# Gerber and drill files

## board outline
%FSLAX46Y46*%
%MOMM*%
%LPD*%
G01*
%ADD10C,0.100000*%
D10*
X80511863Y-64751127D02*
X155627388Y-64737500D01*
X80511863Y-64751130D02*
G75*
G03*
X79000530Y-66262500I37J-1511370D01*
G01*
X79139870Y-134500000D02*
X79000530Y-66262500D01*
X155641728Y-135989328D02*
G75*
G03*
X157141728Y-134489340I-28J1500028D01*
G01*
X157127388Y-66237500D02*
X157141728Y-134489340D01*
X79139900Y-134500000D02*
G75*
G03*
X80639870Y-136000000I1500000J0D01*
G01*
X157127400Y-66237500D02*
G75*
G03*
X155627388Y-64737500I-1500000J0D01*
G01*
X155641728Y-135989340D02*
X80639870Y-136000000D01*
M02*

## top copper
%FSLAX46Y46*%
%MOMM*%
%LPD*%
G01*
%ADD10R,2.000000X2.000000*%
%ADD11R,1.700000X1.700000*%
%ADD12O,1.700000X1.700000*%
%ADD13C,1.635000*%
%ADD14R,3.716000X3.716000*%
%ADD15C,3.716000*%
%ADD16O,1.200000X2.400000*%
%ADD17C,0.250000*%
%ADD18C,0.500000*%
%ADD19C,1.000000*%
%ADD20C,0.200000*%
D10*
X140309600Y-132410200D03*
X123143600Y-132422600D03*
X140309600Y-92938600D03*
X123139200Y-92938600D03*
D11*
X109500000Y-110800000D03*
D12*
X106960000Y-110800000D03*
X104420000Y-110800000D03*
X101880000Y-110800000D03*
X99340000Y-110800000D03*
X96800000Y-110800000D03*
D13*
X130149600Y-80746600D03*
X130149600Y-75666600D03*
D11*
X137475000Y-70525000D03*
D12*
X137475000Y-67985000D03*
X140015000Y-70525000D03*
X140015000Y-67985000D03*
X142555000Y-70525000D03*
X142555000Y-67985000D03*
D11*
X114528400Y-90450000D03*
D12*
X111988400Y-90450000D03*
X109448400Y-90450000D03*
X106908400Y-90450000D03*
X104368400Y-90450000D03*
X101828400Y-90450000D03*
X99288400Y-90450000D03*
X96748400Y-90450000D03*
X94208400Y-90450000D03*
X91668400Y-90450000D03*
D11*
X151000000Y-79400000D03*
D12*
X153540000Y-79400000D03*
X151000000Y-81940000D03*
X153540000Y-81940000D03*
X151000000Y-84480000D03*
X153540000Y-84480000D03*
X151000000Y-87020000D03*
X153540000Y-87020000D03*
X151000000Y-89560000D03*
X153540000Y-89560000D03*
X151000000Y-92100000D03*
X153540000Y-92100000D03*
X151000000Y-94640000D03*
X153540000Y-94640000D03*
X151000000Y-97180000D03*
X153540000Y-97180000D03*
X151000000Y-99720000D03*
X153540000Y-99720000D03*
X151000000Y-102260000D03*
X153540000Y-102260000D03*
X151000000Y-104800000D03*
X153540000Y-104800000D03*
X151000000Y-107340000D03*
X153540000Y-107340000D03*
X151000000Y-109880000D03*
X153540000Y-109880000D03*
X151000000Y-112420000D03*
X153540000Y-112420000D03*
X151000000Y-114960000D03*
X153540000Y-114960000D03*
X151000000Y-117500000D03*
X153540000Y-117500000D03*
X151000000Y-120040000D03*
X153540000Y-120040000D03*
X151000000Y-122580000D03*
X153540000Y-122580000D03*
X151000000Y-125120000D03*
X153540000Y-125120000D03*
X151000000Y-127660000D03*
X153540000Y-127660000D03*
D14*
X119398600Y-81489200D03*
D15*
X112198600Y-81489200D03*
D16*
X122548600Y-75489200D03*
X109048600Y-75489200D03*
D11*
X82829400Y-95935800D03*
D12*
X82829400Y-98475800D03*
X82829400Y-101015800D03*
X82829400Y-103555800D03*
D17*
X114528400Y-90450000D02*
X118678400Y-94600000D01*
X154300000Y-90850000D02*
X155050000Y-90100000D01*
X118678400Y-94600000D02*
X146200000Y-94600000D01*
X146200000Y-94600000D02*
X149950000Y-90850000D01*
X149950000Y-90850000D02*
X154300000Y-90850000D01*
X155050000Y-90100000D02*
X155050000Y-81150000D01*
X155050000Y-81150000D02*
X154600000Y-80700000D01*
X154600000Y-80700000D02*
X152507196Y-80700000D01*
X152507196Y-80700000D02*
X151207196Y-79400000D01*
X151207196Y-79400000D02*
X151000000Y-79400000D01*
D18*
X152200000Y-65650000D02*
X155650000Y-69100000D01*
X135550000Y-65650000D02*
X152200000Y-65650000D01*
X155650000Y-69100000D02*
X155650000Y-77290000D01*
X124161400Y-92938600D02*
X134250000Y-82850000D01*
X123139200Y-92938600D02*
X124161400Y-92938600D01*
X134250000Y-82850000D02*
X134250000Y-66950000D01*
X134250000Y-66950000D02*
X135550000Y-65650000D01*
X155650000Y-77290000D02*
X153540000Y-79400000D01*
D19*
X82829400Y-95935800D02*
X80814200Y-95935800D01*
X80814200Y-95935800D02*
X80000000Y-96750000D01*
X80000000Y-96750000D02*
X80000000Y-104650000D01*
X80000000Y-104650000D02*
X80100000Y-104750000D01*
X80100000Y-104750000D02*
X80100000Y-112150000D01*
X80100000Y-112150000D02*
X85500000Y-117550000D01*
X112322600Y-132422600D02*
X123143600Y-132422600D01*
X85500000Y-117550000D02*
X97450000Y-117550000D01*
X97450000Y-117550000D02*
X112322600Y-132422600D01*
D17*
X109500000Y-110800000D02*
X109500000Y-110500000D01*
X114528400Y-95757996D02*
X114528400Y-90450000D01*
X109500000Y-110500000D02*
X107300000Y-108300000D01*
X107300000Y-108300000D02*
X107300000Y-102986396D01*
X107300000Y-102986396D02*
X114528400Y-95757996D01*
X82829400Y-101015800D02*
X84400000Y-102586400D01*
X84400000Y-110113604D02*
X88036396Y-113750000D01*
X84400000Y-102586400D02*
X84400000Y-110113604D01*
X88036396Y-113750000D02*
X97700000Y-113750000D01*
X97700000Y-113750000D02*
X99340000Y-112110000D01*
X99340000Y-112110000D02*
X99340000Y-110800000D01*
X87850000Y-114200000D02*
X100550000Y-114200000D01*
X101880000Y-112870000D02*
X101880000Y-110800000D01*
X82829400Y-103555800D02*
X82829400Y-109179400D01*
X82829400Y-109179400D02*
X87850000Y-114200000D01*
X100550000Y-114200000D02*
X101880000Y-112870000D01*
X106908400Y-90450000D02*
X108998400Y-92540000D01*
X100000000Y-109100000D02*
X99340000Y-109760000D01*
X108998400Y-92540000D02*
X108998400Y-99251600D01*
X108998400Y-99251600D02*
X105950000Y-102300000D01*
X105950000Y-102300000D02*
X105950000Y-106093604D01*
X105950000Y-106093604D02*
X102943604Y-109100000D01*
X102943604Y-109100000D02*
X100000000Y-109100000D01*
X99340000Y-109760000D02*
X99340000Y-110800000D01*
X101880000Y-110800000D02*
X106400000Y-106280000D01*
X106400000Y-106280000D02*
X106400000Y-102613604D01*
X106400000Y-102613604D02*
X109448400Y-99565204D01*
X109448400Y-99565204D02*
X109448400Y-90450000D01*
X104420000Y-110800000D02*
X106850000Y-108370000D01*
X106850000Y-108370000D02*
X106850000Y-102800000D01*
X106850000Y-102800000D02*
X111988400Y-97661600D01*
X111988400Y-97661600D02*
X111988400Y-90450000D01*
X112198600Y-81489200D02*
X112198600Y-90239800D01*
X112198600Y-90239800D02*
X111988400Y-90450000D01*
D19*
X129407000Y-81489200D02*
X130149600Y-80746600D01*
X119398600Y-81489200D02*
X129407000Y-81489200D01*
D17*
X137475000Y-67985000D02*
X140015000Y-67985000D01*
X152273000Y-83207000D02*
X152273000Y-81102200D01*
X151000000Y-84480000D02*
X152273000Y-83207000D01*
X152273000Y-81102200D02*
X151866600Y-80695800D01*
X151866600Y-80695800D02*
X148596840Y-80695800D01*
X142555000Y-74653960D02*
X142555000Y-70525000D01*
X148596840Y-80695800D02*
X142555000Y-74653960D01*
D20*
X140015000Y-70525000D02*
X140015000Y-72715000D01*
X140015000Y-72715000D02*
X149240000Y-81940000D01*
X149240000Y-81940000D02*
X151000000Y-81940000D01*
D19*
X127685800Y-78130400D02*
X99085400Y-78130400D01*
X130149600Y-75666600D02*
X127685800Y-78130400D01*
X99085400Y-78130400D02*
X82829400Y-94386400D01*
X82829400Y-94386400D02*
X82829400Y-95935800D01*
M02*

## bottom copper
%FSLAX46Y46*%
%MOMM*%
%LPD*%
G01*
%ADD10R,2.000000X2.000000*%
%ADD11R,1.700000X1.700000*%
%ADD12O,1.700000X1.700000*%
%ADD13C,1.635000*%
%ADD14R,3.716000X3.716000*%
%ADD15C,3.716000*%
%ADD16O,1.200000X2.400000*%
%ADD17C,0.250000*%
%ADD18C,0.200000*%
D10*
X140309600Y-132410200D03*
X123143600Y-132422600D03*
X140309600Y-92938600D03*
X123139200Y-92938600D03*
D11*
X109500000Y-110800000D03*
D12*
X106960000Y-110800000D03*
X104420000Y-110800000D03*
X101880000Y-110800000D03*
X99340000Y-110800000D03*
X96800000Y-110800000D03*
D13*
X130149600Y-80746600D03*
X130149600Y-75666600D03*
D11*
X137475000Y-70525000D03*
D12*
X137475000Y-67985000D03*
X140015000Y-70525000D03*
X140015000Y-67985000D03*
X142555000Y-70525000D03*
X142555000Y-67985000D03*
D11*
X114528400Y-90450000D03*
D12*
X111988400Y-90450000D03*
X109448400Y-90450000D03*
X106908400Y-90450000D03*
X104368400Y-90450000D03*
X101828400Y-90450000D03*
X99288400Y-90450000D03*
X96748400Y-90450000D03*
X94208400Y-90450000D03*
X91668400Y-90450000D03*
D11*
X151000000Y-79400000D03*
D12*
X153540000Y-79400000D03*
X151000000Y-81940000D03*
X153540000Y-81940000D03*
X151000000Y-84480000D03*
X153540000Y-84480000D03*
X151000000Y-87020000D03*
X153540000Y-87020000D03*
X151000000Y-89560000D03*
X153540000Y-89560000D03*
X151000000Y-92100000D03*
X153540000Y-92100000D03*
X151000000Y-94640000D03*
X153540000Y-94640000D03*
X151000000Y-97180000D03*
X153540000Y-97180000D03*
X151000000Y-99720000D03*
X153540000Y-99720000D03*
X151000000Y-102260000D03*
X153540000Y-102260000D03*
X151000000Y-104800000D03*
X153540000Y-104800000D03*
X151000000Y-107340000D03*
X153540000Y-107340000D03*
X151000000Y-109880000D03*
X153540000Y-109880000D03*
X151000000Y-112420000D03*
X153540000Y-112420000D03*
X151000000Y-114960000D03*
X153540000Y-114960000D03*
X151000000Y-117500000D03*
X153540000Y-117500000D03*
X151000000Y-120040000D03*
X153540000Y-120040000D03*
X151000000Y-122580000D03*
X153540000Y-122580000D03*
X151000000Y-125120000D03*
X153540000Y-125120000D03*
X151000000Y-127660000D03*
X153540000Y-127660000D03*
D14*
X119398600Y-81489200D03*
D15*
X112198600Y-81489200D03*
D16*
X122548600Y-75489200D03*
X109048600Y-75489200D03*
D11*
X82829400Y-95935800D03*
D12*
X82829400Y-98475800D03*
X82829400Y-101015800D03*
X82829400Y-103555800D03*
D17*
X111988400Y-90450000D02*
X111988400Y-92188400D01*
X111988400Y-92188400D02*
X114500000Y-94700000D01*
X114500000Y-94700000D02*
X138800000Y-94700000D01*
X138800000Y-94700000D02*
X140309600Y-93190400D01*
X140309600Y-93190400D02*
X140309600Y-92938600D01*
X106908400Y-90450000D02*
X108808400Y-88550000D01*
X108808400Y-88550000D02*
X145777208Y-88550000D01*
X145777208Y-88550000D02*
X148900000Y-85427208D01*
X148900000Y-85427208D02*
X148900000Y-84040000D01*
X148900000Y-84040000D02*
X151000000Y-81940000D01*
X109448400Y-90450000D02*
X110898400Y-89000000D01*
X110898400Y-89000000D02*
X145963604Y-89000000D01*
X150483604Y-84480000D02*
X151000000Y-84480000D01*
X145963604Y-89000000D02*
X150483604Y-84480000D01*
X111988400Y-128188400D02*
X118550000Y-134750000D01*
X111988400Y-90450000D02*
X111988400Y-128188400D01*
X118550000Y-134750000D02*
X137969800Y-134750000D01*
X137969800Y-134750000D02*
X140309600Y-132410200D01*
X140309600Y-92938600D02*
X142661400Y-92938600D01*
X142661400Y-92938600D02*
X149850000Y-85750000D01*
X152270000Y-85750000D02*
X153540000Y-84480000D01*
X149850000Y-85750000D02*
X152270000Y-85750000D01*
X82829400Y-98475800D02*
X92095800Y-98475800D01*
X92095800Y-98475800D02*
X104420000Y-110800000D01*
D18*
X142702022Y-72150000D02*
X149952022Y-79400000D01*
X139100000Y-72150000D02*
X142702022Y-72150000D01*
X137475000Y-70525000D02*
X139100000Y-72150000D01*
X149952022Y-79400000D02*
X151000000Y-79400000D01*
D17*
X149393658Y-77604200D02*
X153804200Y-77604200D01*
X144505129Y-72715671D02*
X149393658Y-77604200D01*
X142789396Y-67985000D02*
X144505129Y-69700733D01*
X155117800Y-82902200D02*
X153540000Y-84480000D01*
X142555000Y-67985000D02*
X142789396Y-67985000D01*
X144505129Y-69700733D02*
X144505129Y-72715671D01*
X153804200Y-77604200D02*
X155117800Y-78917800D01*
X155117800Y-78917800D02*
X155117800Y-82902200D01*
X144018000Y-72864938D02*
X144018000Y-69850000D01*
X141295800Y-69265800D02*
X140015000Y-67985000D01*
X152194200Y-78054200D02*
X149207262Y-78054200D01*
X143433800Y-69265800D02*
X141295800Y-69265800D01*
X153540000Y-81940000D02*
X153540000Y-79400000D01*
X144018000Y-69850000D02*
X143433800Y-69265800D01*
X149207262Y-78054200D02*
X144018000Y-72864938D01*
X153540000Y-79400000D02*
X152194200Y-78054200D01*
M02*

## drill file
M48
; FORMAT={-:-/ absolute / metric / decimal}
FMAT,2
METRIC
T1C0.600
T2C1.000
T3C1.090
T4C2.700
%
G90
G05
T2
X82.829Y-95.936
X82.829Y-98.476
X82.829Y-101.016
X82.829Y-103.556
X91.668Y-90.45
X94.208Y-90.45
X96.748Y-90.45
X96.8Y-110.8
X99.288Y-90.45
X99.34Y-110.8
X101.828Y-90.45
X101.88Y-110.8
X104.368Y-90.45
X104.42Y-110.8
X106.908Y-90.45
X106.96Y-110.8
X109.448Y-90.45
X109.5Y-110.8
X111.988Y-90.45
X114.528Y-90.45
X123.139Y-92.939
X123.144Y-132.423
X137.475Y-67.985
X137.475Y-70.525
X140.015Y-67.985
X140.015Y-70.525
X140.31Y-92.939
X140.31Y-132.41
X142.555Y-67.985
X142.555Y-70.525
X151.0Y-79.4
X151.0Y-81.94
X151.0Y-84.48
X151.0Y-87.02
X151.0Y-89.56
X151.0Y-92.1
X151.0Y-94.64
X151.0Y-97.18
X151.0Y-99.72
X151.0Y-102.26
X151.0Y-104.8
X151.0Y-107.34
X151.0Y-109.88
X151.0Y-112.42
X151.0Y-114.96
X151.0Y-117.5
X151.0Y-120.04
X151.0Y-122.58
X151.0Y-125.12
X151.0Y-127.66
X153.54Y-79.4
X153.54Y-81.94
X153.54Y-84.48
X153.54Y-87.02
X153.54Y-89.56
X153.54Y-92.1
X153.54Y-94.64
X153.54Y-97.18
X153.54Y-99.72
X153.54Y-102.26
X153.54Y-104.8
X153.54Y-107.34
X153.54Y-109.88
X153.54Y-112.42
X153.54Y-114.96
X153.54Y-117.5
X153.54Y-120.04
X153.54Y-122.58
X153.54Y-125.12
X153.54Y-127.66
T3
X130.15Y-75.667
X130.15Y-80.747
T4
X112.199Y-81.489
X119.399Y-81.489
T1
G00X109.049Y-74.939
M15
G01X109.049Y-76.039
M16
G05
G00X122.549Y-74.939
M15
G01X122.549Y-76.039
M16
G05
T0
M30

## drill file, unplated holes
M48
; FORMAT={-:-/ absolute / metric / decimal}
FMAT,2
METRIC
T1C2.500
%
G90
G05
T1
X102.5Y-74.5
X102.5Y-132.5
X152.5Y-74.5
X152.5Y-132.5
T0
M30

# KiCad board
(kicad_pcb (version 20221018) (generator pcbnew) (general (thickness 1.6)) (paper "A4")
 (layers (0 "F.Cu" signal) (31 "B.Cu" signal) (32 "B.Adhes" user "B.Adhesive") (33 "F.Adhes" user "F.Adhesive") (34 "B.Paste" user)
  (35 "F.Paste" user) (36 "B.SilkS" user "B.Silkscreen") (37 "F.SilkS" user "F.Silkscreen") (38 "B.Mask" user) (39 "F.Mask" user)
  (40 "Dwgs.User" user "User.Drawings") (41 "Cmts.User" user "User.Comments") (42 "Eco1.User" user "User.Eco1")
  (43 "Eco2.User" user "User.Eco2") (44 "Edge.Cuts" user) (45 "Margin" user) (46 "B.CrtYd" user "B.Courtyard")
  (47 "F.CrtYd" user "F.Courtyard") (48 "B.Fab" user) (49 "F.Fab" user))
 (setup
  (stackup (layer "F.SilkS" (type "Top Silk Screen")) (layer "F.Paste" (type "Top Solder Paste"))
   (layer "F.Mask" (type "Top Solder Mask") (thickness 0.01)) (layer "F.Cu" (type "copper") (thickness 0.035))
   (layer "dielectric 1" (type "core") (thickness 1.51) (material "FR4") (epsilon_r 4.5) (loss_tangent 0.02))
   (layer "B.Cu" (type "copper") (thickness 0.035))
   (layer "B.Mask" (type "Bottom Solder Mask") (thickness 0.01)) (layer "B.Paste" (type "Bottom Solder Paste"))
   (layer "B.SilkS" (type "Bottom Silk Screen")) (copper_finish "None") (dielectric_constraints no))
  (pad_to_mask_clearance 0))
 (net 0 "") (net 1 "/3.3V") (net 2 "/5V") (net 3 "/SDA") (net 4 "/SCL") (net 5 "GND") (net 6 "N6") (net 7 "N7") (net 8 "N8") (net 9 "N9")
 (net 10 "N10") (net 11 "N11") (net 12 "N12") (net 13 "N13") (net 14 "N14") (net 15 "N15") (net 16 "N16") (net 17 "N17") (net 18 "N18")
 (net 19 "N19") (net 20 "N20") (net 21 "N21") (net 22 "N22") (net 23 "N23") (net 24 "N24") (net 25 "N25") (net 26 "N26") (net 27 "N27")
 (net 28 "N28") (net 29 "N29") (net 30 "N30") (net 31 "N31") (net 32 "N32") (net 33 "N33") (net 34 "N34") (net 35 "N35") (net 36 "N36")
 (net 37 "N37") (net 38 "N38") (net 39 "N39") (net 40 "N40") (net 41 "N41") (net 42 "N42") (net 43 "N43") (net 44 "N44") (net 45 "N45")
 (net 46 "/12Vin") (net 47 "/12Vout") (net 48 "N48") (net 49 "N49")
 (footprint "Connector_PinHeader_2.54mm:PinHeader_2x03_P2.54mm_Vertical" (layer "F.Cu") (at 137.475 70.525 90)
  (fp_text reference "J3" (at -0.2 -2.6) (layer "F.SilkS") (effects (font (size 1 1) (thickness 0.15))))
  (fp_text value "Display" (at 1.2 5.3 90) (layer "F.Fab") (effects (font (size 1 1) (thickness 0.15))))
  (pad "1" thru_hole rect (at 0 0 90) (size 1.7 1.7) (drill 1) (layers "*.Cu" "*.Mask") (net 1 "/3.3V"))
  (pad "2" thru_hole oval (at 2.54 0 90) (size 1.7 1.7) (drill 1) (layers "*.Cu" "*.Mask") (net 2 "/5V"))
  (pad "3" thru_hole oval (at 0 2.54 90) (size 1.7 1.7) (drill 1) (layers "*.Cu" "*.Mask") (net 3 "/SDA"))
  (pad "4" thru_hole oval (at 2.54 2.54 90) (size 1.7 1.7) (drill 1) (layers "*.Cu" "*.Mask") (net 2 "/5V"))
  (pad "5" thru_hole oval (at 0 5.08 90) (size 1.7 1.7) (drill 1) (layers "*.Cu" "*.Mask") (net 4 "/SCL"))
  (pad "6" thru_hole oval (at 2.54 5.08 90) (size 1.7 1.7) (drill 1) (layers "*.Cu" "*.Mask") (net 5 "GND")))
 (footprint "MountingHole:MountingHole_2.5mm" (layer "F.Cu") (at 152.5 74.5)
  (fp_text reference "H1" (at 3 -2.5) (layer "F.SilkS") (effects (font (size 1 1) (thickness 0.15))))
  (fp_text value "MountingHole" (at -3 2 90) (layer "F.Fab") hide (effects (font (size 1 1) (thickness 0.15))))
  (pad "" np_thru_hole circle (at 0 0) (size 2.5 2.5) (drill 2.5) (layers "*.Cu" "*.Mask")))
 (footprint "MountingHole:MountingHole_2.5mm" (layer "F.Cu") (at 102.5 74.5)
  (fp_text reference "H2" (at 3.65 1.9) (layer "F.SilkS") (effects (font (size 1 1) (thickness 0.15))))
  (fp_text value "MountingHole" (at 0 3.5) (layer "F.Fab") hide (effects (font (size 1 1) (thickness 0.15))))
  (pad "" np_thru_hole circle (at 0 0) (size 2.5 2.5) (drill 2.5) (layers "*.Cu" "*.Mask")))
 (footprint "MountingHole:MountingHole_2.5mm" (layer "F.Cu") (at 102.5 132.5)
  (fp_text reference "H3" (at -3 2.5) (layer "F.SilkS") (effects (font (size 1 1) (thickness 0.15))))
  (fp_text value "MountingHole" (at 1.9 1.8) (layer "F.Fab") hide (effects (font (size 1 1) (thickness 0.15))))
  (pad "" np_thru_hole circle (at 0 0) (size 2.5 2.5) (drill 2.5) (layers "*.Cu" "*.Mask")))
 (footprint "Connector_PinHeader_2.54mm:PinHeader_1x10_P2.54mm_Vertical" (layer "F.Cu") (at 114.5284 90.45 -90)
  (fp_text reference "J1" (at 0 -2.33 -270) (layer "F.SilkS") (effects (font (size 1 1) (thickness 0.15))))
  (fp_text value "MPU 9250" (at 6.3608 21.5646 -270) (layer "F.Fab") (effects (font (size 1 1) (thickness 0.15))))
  (pad "1" thru_hole rect (at 0 0 270) (size 1.7 1.7) (drill 1) (layers "*.Cu" "*.Mask") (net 1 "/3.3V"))
  (pad "2" thru_hole oval (at 0 2.54 270) (size 1.7 1.7) (drill 1) (layers "*.Cu" "*.Mask") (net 5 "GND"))
  (pad "3" thru_hole oval (at 0 5.08 270) (size 1.7 1.7) (drill 1) (layers "*.Cu" "*.Mask") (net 4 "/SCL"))
  (pad "4" thru_hole oval (at 0 7.62 270) (size 1.7 1.7) (drill 1) (layers "*.Cu" "*.Mask") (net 3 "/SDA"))
  (pad "5" thru_hole oval (at 0 10.16 270) (size 1.7 1.7) (drill 1) (layers "*.Cu" "*.Mask") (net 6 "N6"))
  (pad "6" thru_hole oval (at 0 12.7 270) (size 1.7 1.7) (drill 1) (layers "*.Cu" "*.Mask") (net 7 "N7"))
  (pad "7" thru_hole oval (at 0 15.24 270) (size 1.7 1.7) (drill 1) (layers "*.Cu" "*.Mask") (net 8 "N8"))
  (pad "8" thru_hole oval (at 0 17.78 270) (size 1.7 1.7) (drill 1) (layers "*.Cu" "*.Mask") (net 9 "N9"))
  (pad "9" thru_hole oval (at 0 20.32 270) (size 1.7 1.7) (drill 1) (layers "*.Cu" "*.Mask") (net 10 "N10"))
  (pad "10" thru_hole oval (at 0 22.86 270) (size 1.7 1.7) (drill 1) (layers "*.Cu" "*.Mask") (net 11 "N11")))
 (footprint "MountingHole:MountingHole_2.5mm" (layer "F.Cu") (at 152.5 132.5)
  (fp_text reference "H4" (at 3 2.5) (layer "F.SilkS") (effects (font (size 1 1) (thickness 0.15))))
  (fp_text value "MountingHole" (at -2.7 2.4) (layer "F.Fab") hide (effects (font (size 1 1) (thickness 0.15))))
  (pad "" np_thru_hole circle (at 0 0) (size 2.5 2.5) (drill 2.5) (layers "*.Cu" "*.Mask")))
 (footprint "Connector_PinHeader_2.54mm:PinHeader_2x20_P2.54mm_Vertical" (layer "F.Cu") (at 151 79.4)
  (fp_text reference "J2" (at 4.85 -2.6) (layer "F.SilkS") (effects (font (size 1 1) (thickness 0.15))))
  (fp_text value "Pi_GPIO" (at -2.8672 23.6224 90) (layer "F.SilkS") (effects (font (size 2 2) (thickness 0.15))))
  (pad "1" thru_hole rect (at 0 0) (size 1.7 1.7) (drill 1) (layers "*.Cu" "*.Mask") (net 1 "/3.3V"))
  (pad "2" thru_hole oval (at 2.54 0) (size 1.7 1.7) (drill 1) (layers "*.Cu" "*.Mask") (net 2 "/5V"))
  (pad "3" thru_hole oval (at 0 2.54) (size 1.7 1.7) (drill 1) (layers "*.Cu" "*.Mask") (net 3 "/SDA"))
  (pad "4" thru_hole oval (at 2.54 2.54) (size 1.7 1.7) (drill 1) (layers "*.Cu" "*.Mask") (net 2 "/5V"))
  (pad "5" thru_hole oval (at 0 5.08) (size 1.7 1.7) (drill 1) (layers "*.Cu" "*.Mask") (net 4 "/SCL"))
  (pad "6" thru_hole oval (at 2.54 5.08) (size 1.7 1.7) (drill 1) (layers "*.Cu" "*.Mask") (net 5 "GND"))
  (pad "7" thru_hole oval (at 0 7.62) (size 1.7 1.7) (drill 1) (layers "*.Cu" "*.Mask") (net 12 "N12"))
  (pad "8" thru_hole oval (at 2.54 7.62) (size 1.7 1.7) (drill 1) (layers "*.Cu" "*.Mask") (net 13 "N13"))
  (pad "9" thru_hole oval (at 0 10.16) (size 1.7 1.7) (drill 1) (layers "*.Cu" "*.Mask") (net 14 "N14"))
  (pad "10" thru_hole oval (at 2.54 10.16) (size 1.7 1.7) (drill 1) (layers "*.Cu" "*.Mask") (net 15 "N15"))
  (pad "11" thru_hole oval (at 0 12.7) (size 1.7 1.7) (drill 1) (layers "*.Cu" "*.Mask") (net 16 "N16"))
  (pad "12" thru_hole oval (at 2.54 12.7) (size 1.7 1.7) (drill 1) (layers "*.Cu" "*.Mask") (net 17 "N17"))
  (pad "13" thru_hole oval (at 0 15.24) (size 1.7 1.7) (drill 1) (layers "*.Cu" "*.Mask") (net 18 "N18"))
  (pad "14" thru_hole oval (at 2.54 15.24) (size 1.7 1.7) (drill 1) (layers "*.Cu" "*.Mask") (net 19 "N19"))
  (pad "15" thru_hole oval (at 0 17.78) (size 1.7 1.7) (drill 1) (layers "*.Cu" "*.Mask") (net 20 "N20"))
  (pad "16" thru_hole oval (at 2.54 17.78) (size 1.7 1.7) (drill 1) (layers "*.Cu" "*.Mask") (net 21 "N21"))
  (pad "17" thru_hole oval (at 0 20.32) (size 1.7 1.7) (drill 1) (layers "*.Cu" "*.Mask") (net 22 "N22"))
  (pad "18" thru_hole oval (at 2.54 20.32) (size 1.7 1.7) (drill 1) (layers "*.Cu" "*.Mask") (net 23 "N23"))
  (pad "19" thru_hole oval (at 0 22.86) (size 1.7 1.7) (drill 1) (layers "*.Cu" "*.Mask") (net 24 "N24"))
  (pad "20" thru_hole oval (at 2.54 22.86) (size 1.7 1.7) (drill 1) (layers "*.Cu" "*.Mask") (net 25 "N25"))
  (pad "21" thru_hole oval (at 0 25.4) (size 1.7 1.7) (drill 1) (layers "*.Cu" "*.Mask") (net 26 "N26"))
  (pad "22" thru_hole oval (at 2.54 25.4) (size 1.7 1.7) (drill 1) (layers "*.Cu" "*.Mask") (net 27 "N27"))
  (pad "23" thru_hole oval (at 0 27.94) (size 1.7 1.7) (drill 1) (layers "*.Cu" "*.Mask") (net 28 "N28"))
  (pad "24" thru_hole oval (at 2.54 27.94) (size 1.7 1.7) (drill 1) (layers "*.Cu" "*.Mask") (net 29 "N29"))
  (pad "25" thru_hole oval (at 0 30.48) (size 1.7 1.7) (drill 1) (layers "*.Cu" "*.Mask") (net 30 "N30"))
  (pad "26" thru_hole oval (at 2.54 30.48) (size 1.7 1.7) (drill 1) (layers "*.Cu" "*.Mask") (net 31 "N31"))
  (pad "27" thru_hole oval (at 0 33.02) (size 1.7 1.7) (drill 1) (layers "*.Cu" "*.Mask") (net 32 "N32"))
  (pad "28" thru_hole oval (at 2.54 33.02) (size 1.7 1.7) (drill 1) (layers "*.Cu" "*.Mask") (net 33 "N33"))
  (pad "29" thru_hole oval (at 0 35.56) (size 1.7 1.7) (drill 1) (layers "*.Cu" "*.Mask") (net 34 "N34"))
  (pad "30" thru_hole oval (at 2.54 35.56) (size 1.7 1.7) (drill 1) (layers "*.Cu" "*.Mask") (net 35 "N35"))
  (pad "31" thru_hole oval (at 0 38.1) (size 1.7 1.7) (drill 1) (layers "*.Cu" "*.Mask") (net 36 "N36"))
  (pad "32" thru_hole oval (at 2.54 38.1) (size 1.7 1.7) (drill 1) (layers "*.Cu" "*.Mask") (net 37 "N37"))
  (pad "33" thru_hole oval (at 0 40.64) (size 1.7 1.7) (drill 1) (layers "*.Cu" "*.Mask") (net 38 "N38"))
  (pad "34" thru_hole oval (at 2.54 40.64) (size 1.7 1.7) (drill 1) (layers "*.Cu" "*.Mask") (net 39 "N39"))
  (pad "35" thru_hole oval (at 0 43.18) (size 1.7 1.7) (drill 1) (layers "*.Cu" "*.Mask") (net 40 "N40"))
  (pad "36" thru_hole oval (at 2.54 43.18) (size 1.7 1.7) (drill 1) (layers "*.Cu" "*.Mask") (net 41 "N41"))
  (pad "37" thru_hole oval (at 0 45.72) (size 1.7 1.7) (drill 1) (layers "*.Cu" "*.Mask") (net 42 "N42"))
  (pad "38" thru_hole oval (at 2.54 45.72) (size 1.7 1.7) (drill 1) (layers "*.Cu" "*.Mask") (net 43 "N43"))
  (pad "39" thru_hole oval (at 0 48.26) (size 1.7 1.7) (drill 1) (layers "*.Cu" "*.Mask") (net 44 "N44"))
  (pad "40" thru_hole oval (at 2.54 48.26) (size 1.7 1.7) (drill 1) (layers "*.Cu" "*.Mask") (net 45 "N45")))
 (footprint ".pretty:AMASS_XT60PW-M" (layer "F.Cu") (at 115.7986 75.4892)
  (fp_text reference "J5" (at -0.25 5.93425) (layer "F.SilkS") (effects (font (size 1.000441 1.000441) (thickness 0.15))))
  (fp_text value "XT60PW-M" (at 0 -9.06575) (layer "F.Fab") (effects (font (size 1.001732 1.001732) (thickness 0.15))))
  (pad "1" thru_hole rect (at 3.6 6) (size 3.716 3.716) (drill 2.7) (layers "*.Cu" "*.Mask") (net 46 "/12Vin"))
  (pad "2" thru_hole circle (at -3.6 6) (size 3.716 3.716) (drill 2.7) (layers "*.Cu" "*.Mask") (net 5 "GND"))
  (pad "S1" thru_hole oval (at 6.75 0) (size 1.2 2.4) (drill oval 0.6 1.7) (layers "*.Cu" "*.Mask"))
  (pad "S2" thru_hole oval (at -6.75 0) (size 1.2 2.4) (drill oval 0.6 1.7) (layers "*.Cu" "*.Mask")))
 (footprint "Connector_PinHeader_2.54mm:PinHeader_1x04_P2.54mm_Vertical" (layer "F.Cu") (at 82.8294 95.9358)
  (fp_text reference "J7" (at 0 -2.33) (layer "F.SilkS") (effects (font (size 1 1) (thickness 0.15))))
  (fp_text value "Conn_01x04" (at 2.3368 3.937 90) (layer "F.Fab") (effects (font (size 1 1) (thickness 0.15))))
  (pad "1" thru_hole rect (at 0 0) (size 1.7 1.7) (drill 1) (layers "*.Cu" "*.Mask") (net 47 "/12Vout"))
  (pad "2" thru_hole oval (at 0 2.54) (size 1.7 1.7) (drill 1) (layers "*.Cu" "*.Mask") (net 5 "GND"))
  (pad "3" thru_hole oval (at 0 5.08) (size 1.7 1.7) (drill 1) (layers "*.Cu" "*.Mask") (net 3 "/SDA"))
  (pad "4" thru_hole oval (at 0 7.62) (size 1.7 1.7) (drill 1) (layers "*.Cu" "*.Mask") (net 4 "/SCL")))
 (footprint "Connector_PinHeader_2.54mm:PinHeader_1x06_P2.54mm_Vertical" (layer "F.Cu") (at 109.5 110.8 -90)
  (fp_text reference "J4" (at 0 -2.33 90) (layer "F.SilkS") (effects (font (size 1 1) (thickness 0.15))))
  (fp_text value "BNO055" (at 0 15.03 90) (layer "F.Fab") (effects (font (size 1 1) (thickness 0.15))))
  (pad "1" thru_hole rect (at 0 0 270) (size 1.7 1.7) (drill 1) (layers "*.Cu" "*.Mask") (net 1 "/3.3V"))
  (pad "2" thru_hole oval (at 0 2.54 270) (size 1.7 1.7) (drill 1) (layers "*.Cu" "*.Mask") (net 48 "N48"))
  (pad "3" thru_hole oval (at 0 5.08 270) (size 1.7 1.7) (drill 1) (layers "*.Cu" "*.Mask") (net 5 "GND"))
  (pad "4" thru_hole oval (at 0 7.62 270) (size 1.7 1.7) (drill 1) (layers "*.Cu" "*.Mask") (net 4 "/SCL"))
  (pad "5" thru_hole oval (at 0 10.16 270) (size 1.7 1.7) (drill 1) (layers "*.Cu" "*.Mask") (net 3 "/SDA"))
  (pad "6" thru_hole oval (at 0 12.7 270) (size 1.7 1.7) (drill 1) (layers "*.Cu" "*.Mask") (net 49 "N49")))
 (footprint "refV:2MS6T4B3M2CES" (layer "F.Cu") (at 130.1496 80.7466)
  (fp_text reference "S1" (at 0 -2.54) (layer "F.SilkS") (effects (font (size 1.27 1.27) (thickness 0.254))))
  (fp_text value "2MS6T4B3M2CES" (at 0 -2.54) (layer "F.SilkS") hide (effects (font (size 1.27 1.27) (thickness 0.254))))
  (pad "1" thru_hole circle (at 0 0) (size 1.635 1.635) (drill 1.09) (layers "*.Cu" "*.Mask") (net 46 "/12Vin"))
  (pad "3" thru_hole circle (at 0 -5.08) (size 1.635 1.635) (drill 1.09) (layers "*.Cu" "*.Mask") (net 47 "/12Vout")))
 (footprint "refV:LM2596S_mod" (layer "B.Cu") (at 145.6436 123.6726 90)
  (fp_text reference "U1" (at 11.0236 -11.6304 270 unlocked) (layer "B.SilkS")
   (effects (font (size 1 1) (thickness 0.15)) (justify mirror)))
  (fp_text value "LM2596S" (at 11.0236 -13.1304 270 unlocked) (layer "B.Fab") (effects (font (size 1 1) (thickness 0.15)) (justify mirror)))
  (pad "1" thru_hole rect (at -8.7376 -5.334 90) (size 2 2) (drill 1) (layers "*.Cu" "*.Mask") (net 5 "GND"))
  (pad "2" thru_hole rect (at -8.75 -22.5 90) (size 2 2) (drill 1) (layers "*.Cu" "*.Mask") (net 47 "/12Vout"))
  (pad "3" thru_hole rect (at 30.734 -5.334 90) (size 2 2) (drill 1) (layers "*.Cu" "*.Mask") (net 5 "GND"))
  (pad "4" thru_hole rect (at 30.734 -22.5044 90) (size 2 2) (drill 1) (layers "*.Cu" "*.Mask") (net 2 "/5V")))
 (gr_line (start 80.511863 64.751127) (end 155.627388 64.7375) (stroke (width 0.1) (type solid)) (layer "Edge.Cuts"))
 (gr_arc (start 79.00053 66.2625) (mid 79.443187 65.193812) (end 80.511863 64.751127) (stroke (width 0.1) (type solid)) (layer "Edge.Cuts"))
 (gr_line (start 79.13987 134.5) (end 79.00053 66.2625) (stroke (width 0.1) (type solid)) (layer "Edge.Cuts"))
 (gr_arc (start 157.141728 134.48934) (mid 156.702376 135.549988) (end 155.641728 135.98934) (stroke (width 0.1) (type solid))
  (layer "Edge.Cuts"))
 (gr_line (start 157.127388 66.2375) (end 157.141728 134.48934) (stroke (width 0.1) (type solid)) (layer "Edge.Cuts"))
 (gr_arc (start 80.63987 136) (mid 79.57921 135.56066) (end 79.13987 134.5) (stroke (width 0.1) (type solid)) (layer "Edge.Cuts"))
 (gr_arc (start 155.627388 64.7375) (mid 156.688048 65.17684) (end 157.127388 66.2375) (stroke (width 0.1) (type solid)) (layer "Edge.Cuts"))
 (gr_line (start 155.641728 135.98934) (end 80.63987 136) (stroke (width 0.1) (type solid)) (layer "Edge.Cuts"))
 (segment (start 129.407 81.4892) (end 130.1496 80.7466) (width 1) (layer "F.Cu") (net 46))
 (segment (start 119.3986 81.4892) (end 129.407 81.4892) (width 1) (layer "F.Cu") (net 46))
 (segment (start 107.3 108.3) (end 107.3 102.986396) (width 0.25) (layer "F.Cu") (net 1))
 (segment (start 154.3 90.85) (end 155.05 90.1) (width 0.25) (layer "F.Cu") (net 1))
 (segment (start 109.5 110.5) (end 107.3 108.3) (width 0.25) (layer "F.Cu") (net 1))
 (segment (start 151.207196 79.4) (end 151 79.4) (width 0.25) (layer "F.Cu") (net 1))
 (segment (start 155.05 81.15) (end 154.6 80.7) (width 0.25) (layer "F.Cu") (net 1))
 (segment (start 155.05 90.1) (end 155.05 81.15) (width 0.25) (layer "F.Cu") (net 1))
 (segment (start 146.2 94.6) (end 149.95 90.85) (width 0.25) (layer "F.Cu") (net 1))
 (segment (start 114.5284 95.757996) (end 114.5284 90.45) (width 0.25) (layer "F.Cu") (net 1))
 (segment (start 114.5284 90.45) (end 118.6784 94.6) (width 0.25) (layer "F.Cu") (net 1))
 (segment (start 152.507196 80.7) (end 151.207196 79.4) (width 0.25) (layer "F.Cu") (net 1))
 (segment (start 154.6 80.7) (end 152.507196 80.7) (width 0.25) (layer "F.Cu") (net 1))
 (segment (start 109.5 110.8) (end 109.5 110.5) (width 0.25) (layer "F.Cu") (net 1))
 (segment (start 107.3 102.986396) (end 114.5284 95.757996) (width 0.25) (layer "F.Cu") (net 1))
 (segment (start 118.6784 94.6) (end 146.2 94.6) (width 0.25) (layer "F.Cu") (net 1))
 (segment (start 149.95 90.85) (end 154.3 90.85) (width 0.25) (layer "F.Cu") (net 1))
 (segment (start 142.702022 72.15) (end 149.952022 79.4) (width 0.2) (layer "B.Cu") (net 1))
 (segment (start 139.1 72.15) (end 142.702022 72.15) (width 0.2) (layer "B.Cu") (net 1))
 (segment (start 137.475 70.525) (end 139.1 72.15) (width 0.2) (layer "B.Cu") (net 1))
 (segment (start 149.952022 79.4) (end 151 79.4) (width 0.2) (layer "B.Cu") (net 1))
 (segment (start 112.1986 90.2398) (end 111.9884 90.45) (width 0.25) (layer "F.Cu") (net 5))
 (segment (start 112.1986 81.4892) (end 112.1986 90.2398) (width 0.25) (layer "F.Cu") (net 5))
 (segment (start 104.42 110.8) (end 106.85 108.37) (width 0.25) (layer "F.Cu") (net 5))
 (segment (start 106.85 102.8) (end 111.9884 97.6616) (width 0.25) (layer "F.Cu") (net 5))
 (segment (start 106.85 108.37) (end 106.85 102.8) (width 0.25) (layer "F.Cu") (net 5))
 (segment (start 111.9884 97.6616) (end 111.9884 90.45) (width 0.25) (layer "F.Cu") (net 5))
 (segment (start 118.55 134.75) (end 137.9698 134.75) (width 0.25) (layer "B.Cu") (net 5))
 (segment (start 149.393658 77.6042) (end 153.8042 77.6042) (width 0.25) (layer "B.Cu") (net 5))
 (segment (start 92.0958 98.4758) (end 104.42 110.8) (width 0.25) (layer "B.Cu") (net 5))
 (segment (start 140.3096 92.9386) (end 142.6614 92.9386) (width 0.25) (layer "B.Cu") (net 5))
 (segment (start 140.3096 93.1904) (end 140.3096 92.9386) (width 0.25) (layer "B.Cu") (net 5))
 (segment (start 137.9698 134.75) (end 140.3096 132.4102) (width 0.25) (layer "B.Cu") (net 5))
 (segment (start 144.505129 72.715671) (end 149.393658 77.6042) (width 0.25) (layer "B.Cu") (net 5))
 (segment (start 142.789396 67.985) (end 144.505129 69.700733) (width 0.25) (layer "B.Cu") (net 5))
 (segment (start 155.1178 82.9022) (end 153.54 84.48) (width 0.25) (layer "B.Cu") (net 5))
 (segment (start 114.5 94.7) (end 138.8 94.7) (width 0.25) (layer "B.Cu") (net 5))
 (segment (start 142.555 67.985) (end 142.789396 67.985) (width 0.25) (layer "B.Cu") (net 5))
 (segment (start 111.9884 90.45) (end 111.9884 128.1884) (width 0.25) (layer "B.Cu") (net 5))
 (segment (start 149.85 85.75) (end 152.27 85.75) (width 0.25) (layer "B.Cu") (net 5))
 (segment (start 111.9884 128.1884) (end 118.55 134.75) (width 0.25) (layer "B.Cu") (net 5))
 (segment (start 152.27 85.75) (end 153.54 84.48) (width 0.25) (layer "B.Cu") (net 5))
 (segment (start 82.8294 98.4758) (end 92.0958 98.4758) (width 0.25) (layer "B.Cu") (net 5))
 (segment (start 142.6614 92.9386) (end 149.85 85.75) (width 0.25) (layer "B.Cu") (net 5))
 (segment (start 144.505129 69.700733) (end 144.505129 72.715671) (width 0.25) (layer "B.Cu") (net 5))
 (segment (start 153.8042 77.6042) (end 155.1178 78.9178) (width 0.25) (layer "B.Cu") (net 5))
 (segment (start 155.1178 78.9178) (end 155.1178 82.9022) (width 0.25) (layer "B.Cu") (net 5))
 (segment (start 111.9884 92.1884) (end 114.5 94.7) (width 0.25) (layer "B.Cu") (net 5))
 (segment (start 111.9884 90.45) (end 111.9884 92.1884) (width 0.25) (layer "B.Cu") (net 5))
 (segment (start 138.8 94.7) (end 140.3096 93.1904) (width 0.25) (layer "B.Cu") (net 5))
 (segment (start 123.1392 92.9386) (end 124.1614 92.9386) (width 0.5) (layer "F.Cu") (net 2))
 (segment (start 155.65 69.1) (end 155.65 77.29) (width 0.5) (layer "F.Cu") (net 2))
 (segment (start 152.2 65.65) (end 155.65 69.1) (width 0.5) (layer "F.Cu") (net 2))
 (segment (start 137.475 67.985) (end 140.015 67.985) (width 0.25) (layer "F.Cu") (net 2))
 (segment (start 134.25 82.85) (end 134.25 66.95) (width 0.5) (layer "F.Cu") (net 2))
 (segment (start 134.25 66.95) (end 135.55 65.65) (width 0.5) (layer "F.Cu") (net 2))
 (segment (start 155.65 77.29) (end 153.54 79.4) (width 0.5) (layer "F.Cu") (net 2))
 (segment (start 135.55 65.65) (end 152.2 65.65) (width 0.5) (layer "F.Cu") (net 2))
 (segment (start 124.1614 92.9386) (end 134.25 82.85) (width 0.5) (layer "F.Cu") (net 2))
 (segment (start 144.018 72.864938) (end 144.018 69.85) (width 0.25) (layer "B.Cu") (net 2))
 (segment (start 141.2958 69.2658) (end 140.015 67.985) (width 0.25) (layer "B.Cu") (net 2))
 (segment (start 152.1942 78.0542) (end 149.207262 78.0542) (width 0.25) (layer "B.Cu") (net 2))
 (segment (start 143.4338 69.2658) (end 141.2958 69.2658) (width 0.25) (layer "B.Cu") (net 2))
 (segment (start 153.54 81.94) (end 153.54 79.4) (width 0.25) (layer "B.Cu") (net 2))
 (segment (start 144.018 69.85) (end 143.4338 69.2658) (width 0.25) (layer "B.Cu") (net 2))
 (segment (start 149.207262 78.0542) (end 144.018 72.864938) (width 0.25) (layer "B.Cu") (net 2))
 (segment (start 153.54 79.4) (end 152.1942 78.0542) (width 0.25) (layer "B.Cu") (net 2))
 (segment (start 101.88 112.87) (end 101.88 110.8) (width 0.25) (layer "F.Cu") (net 4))
 (segment (start 152.273 83.207) (end 152.273 81.1022) (width 0.25) (layer "F.Cu") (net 4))
 (segment (start 82.8294 109.1794) (end 87.85 114.2) (width 0.25) (layer "F.Cu") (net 4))
 (segment (start 151 84.48) (end 152.273 83.207) (width 0.25) (layer "F.Cu") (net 4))
 (segment (start 82.8294 103.5558) (end 82.8294 109.1794) (width 0.25) (layer "F.Cu") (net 4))
 (segment (start 152.273 81.1022) (end 151.8666 80.6958) (width 0.25) (layer "F.Cu") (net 4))
 (segment (start 100.55 114.2) (end 101.88 112.87) (width 0.25) (layer "F.Cu") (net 4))
 (segment (start 109.4484 99.565204) (end 109.4484 90.45) (width 0.25) (layer "F.Cu") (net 4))
 (segment (start 151.8666 80.6958) (end 148.59684 80.6958) (width 0.25) (layer "F.Cu") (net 4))
 (segment (start 142.555 74.65396) (end 142.555 70.525) (width 0.25) (layer "F.Cu") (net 4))
 (segment (start 106.4 102.613604) (end 109.4484 99.565204) (width 0.25) (layer "F.Cu") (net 4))
 (segment (start 101.88 110.8) (end 106.4 106.28) (width 0.25) (layer "F.Cu") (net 4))
 (segment (start 148.59684 80.6958) (end 142.555 74.65396) (width 0.25) (layer "F.Cu") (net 4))
 (segment (start 106.4 106.28) (end 106.4 102.613604) (width 0.25) (layer "F.Cu") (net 4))
 (segment (start 87.85 114.2) (end 100.55 114.2) (width 0.25) (layer "F.Cu") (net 4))
 (segment (start 109.4484 90.45) (end 110.8984 89) (width 0.25) (layer "B.Cu") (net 4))
 (segment (start 150.483604 84.48) (end 151 84.48) (width 0.25) (layer "B.Cu") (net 4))
 (segment (start 145.963604 89) (end 150.483604 84.48) (width 0.25) (layer "B.Cu") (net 4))
 (segment (start 110.8984 89) (end 145.963604 89) (width 0.25) (layer "B.Cu") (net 4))
 (segment (start 140.015 70.525) (end 140.015 72.715) (width 0.2) (layer "F.Cu") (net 3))
 (segment (start 82.8294 101.0158) (end 84.4 102.5864) (width 0.25) (layer "F.Cu") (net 3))
 (segment (start 99.34 112.11) (end 99.34 110.8) (width 0.25) (layer "F.Cu") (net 3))
 (segment (start 84.4 110.113604) (end 88.036396 113.75) (width 0.25) (layer "F.Cu") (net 3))
 (segment (start 140.015 72.715) (end 149.24 81.94) (width 0.2) (layer "F.Cu") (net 3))
 (segment (start 97.7 113.75) (end 99.34 112.11) (width 0.25) (layer "F.Cu") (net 3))
 (segment (start 105.95 102.3) (end 105.95 106.093604) (width 0.25) (layer "F.Cu") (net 3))
 (segment (start 108.9984 92.54) (end 108.9984 99.2516) (width 0.25) (layer "F.Cu") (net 3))
 (segment (start 99.34 109.76) (end 99.34 110.8) (width 0.25) (layer "F.Cu") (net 3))
 (segment (start 102.943604 109.1) (end 100 109.1) (width 0.25) (layer "F.Cu") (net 3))
 (segment (start 100 109.1) (end 99.34 109.76) (width 0.25) (layer "F.Cu") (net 3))
 (segment (start 84.4 102.5864) (end 84.4 110.113604) (width 0.25) (layer "F.Cu") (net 3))
 (segment (start 106.9084 90.45) (end 108.9984 92.54) (width 0.25) (layer "F.Cu") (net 3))
 (segment (start 88.036396 113.75) (end 97.7 113.75) (width 0.25) (layer "F.Cu") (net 3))
 (segment (start 108.9984 99.2516) (end 105.95 102.3) (width 0.25) (layer "F.Cu") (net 3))
 (segment (start 105.95 106.093604) (end 102.943604 109.1) (width 0.25) (layer "F.Cu") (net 3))
 (segment (start 149.24 81.94) (end 151 81.94) (width 0.2) (layer "F.Cu") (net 3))
 (segment (start 145.777208 88.55) (end 148.9 85.427208) (width 0.25) (layer "B.Cu") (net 3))
 (segment (start 108.8084 88.55) (end 145.777208 88.55) (width 0.25) (layer "B.Cu") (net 3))
 (segment (start 148.9 84.04) (end 151 81.94) (width 0.25) (layer "B.Cu") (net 3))
 (segment (start 106.9084 90.45) (end 108.8084 88.55) (width 0.25) (layer "B.Cu") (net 3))
 (segment (start 148.9 85.427208) (end 148.9 84.04) (width 0.25) (layer "B.Cu") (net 3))
 (segment (start 127.6858 78.1304) (end 99.0854 78.1304) (width 1) (layer "F.Cu") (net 47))
 (segment (start 85.5 117.55) (end 97.45 117.55) (width 1) (layer "F.Cu") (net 47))
 (segment (start 130.1496 75.6666) (end 127.6858 78.1304) (width 1) (layer "F.Cu") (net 47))
 (segment (start 80.1 112.15) (end 85.5 117.55) (width 1) (layer "F.Cu") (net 47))
 (segment (start 80.8142 95.9358) (end 80 96.75) (width 1) (layer "F.Cu") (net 47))
 (segment (start 80.1 104.75) (end 80.1 112.15) (width 1) (layer "F.Cu") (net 47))
 (segment (start 80 104.65) (end 80.1 104.75) (width 1) (layer "F.Cu") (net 47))
 (segment (start 112.3226 132.4226) (end 123.1436 132.4226) (width 1) (layer "F.Cu") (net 47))
 (segment (start 99.0854 78.1304) (end 82.8294 94.3864) (width 1) (layer "F.Cu") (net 47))
 (segment (start 82.8294 95.9358) (end 80.8142 95.9358) (width 1) (layer "F.Cu") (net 47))
 (segment (start 82.8294 94.3864) (end 82.8294 95.9358) (width 1) (layer "F.Cu") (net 47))
 (segment (start 97.45 117.55) (end 112.3226 132.4226) (width 1) (layer "F.Cu") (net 47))
 (segment (start 80 96.75) (end 80 104.65) (width 1) (layer "F.Cu") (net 47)))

